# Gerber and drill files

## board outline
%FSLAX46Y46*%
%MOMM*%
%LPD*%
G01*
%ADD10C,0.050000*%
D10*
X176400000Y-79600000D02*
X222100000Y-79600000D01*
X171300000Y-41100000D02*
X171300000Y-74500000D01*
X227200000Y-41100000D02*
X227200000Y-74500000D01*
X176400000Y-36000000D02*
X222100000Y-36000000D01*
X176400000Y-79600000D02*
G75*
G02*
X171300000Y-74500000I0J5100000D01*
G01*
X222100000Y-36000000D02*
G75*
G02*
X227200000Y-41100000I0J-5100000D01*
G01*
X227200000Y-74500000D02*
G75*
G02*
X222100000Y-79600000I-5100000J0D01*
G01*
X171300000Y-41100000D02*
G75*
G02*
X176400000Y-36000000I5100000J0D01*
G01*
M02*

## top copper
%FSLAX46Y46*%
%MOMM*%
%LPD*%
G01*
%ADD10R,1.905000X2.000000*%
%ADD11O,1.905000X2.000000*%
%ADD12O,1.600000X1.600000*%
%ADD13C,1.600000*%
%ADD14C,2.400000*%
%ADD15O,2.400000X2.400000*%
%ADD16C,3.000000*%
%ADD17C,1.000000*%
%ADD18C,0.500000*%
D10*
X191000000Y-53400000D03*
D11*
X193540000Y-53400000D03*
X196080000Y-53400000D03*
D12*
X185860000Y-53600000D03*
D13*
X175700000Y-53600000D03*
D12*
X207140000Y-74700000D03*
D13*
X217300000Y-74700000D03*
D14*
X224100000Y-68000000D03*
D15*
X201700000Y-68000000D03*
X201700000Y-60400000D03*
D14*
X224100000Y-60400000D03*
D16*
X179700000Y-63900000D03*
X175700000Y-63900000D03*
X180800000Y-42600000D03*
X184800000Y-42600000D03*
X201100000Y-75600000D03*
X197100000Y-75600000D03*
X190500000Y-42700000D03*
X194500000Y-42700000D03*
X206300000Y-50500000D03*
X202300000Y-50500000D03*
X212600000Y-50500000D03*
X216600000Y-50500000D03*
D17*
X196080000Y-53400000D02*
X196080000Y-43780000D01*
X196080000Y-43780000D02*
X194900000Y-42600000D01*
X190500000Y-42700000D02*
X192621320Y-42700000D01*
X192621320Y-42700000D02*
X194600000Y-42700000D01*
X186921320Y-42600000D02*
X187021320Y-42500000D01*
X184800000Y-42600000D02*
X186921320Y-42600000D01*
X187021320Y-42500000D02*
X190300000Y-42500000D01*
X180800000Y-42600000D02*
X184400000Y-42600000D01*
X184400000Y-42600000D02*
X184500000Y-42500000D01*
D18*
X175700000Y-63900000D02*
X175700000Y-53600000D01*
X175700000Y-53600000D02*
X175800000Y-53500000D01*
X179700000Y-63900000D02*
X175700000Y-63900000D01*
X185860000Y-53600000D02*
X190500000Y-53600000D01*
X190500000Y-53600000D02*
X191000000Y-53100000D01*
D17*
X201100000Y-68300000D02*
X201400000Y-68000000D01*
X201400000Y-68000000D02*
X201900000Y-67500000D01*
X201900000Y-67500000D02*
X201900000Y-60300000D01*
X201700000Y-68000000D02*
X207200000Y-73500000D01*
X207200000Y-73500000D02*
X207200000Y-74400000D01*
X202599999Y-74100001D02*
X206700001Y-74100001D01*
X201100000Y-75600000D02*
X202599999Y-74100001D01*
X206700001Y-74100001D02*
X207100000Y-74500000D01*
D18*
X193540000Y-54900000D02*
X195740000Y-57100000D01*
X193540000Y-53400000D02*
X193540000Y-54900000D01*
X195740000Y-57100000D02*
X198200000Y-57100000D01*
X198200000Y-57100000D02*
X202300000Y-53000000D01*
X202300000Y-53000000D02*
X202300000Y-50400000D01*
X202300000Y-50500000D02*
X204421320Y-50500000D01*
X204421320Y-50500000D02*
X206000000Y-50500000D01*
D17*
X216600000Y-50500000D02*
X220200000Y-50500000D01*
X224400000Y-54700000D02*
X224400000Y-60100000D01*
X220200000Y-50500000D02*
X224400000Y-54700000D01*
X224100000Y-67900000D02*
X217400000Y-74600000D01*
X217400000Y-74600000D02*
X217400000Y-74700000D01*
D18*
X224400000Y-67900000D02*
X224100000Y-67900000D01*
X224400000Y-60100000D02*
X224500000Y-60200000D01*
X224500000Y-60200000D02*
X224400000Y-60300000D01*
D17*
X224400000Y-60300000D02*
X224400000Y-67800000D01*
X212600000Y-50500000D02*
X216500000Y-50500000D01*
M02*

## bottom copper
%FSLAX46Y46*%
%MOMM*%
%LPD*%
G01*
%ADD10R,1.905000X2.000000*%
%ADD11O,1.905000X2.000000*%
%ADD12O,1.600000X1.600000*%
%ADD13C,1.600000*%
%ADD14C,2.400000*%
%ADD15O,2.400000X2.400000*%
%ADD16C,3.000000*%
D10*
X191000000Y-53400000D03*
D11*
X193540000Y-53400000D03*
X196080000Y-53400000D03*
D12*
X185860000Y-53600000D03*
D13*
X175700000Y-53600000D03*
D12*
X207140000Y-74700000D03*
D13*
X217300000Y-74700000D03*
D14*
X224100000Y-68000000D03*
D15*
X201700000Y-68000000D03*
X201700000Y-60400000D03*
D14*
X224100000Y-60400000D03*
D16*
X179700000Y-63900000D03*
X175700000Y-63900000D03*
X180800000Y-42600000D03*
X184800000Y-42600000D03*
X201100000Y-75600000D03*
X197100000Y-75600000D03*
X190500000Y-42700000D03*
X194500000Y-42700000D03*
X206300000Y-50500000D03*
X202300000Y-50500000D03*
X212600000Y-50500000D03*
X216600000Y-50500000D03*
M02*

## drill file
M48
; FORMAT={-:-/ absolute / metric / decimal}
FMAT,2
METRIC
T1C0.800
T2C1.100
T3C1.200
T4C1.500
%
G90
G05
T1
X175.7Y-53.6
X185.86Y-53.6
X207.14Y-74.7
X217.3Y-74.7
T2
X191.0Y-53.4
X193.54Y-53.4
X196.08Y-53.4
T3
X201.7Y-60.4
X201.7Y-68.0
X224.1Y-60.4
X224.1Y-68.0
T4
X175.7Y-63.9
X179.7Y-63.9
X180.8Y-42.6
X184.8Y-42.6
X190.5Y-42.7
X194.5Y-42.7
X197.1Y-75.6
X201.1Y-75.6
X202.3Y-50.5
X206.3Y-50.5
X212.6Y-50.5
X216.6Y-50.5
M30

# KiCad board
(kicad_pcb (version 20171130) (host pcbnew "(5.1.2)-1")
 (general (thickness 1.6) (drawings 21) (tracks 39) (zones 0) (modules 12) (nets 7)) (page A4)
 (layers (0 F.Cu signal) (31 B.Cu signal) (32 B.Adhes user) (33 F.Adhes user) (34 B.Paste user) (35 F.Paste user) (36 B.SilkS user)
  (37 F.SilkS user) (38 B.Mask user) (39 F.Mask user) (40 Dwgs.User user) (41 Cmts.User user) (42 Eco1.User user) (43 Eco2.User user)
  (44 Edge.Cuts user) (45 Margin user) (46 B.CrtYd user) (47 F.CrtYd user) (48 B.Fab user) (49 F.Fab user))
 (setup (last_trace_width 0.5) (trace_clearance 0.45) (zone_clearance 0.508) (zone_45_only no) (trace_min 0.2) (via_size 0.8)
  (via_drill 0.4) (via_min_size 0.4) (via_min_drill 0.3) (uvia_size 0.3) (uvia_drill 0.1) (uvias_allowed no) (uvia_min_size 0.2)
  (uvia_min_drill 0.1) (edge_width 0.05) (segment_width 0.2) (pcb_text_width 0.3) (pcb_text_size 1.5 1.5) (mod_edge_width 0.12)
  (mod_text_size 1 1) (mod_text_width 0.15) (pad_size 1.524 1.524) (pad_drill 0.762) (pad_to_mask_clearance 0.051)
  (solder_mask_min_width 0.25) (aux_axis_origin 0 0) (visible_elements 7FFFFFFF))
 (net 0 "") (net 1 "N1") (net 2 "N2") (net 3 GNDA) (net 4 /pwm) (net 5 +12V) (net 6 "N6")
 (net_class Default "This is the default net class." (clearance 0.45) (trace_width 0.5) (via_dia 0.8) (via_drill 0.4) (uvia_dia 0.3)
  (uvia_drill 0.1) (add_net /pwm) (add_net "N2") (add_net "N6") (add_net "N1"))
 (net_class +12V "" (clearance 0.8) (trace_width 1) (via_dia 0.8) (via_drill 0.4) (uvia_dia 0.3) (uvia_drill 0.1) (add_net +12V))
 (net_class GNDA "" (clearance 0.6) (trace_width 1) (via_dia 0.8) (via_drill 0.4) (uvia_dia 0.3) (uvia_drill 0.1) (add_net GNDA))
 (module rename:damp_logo (layer F.Cu) (at 217.8 40.1)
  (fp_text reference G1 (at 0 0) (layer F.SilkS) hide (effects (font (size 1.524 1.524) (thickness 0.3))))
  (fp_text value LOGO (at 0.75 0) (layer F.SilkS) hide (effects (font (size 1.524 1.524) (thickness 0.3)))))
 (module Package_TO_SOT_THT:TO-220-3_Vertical (layer F.Cu) (at 191 53.4)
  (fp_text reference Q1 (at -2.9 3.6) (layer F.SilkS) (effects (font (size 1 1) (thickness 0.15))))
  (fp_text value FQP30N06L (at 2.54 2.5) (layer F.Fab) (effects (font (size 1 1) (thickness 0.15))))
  (pad 1 thru_hole rect (at 0 0) (size 1.905 2) (drill 1.1) (layers *.Cu *.Mask) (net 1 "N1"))
  (pad 2 thru_hole oval (at 2.54 0) (size 1.905 2) (drill 1.1) (layers *.Cu *.Mask) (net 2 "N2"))
  (pad 3 thru_hole oval (at 5.08 0) (size 1.905 2) (drill 1.1) (layers *.Cu *.Mask) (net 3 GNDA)))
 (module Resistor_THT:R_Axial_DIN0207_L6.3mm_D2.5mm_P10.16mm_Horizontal (layer F.Cu) (at 175.7 53.6)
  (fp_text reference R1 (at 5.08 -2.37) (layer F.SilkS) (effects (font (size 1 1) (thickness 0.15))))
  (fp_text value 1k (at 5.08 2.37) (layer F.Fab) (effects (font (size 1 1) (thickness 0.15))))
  (pad 2 thru_hole oval (at 10.16 0) (size 1.6 1.6) (drill 0.8) (layers *.Cu *.Mask) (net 1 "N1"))
  (pad 1 thru_hole circle (at 0 0) (size 1.6 1.6) (drill 0.8) (layers *.Cu *.Mask) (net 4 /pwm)))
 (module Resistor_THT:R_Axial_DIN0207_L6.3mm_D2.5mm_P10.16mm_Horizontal (layer F.Cu) (at 217.3 74.7 180)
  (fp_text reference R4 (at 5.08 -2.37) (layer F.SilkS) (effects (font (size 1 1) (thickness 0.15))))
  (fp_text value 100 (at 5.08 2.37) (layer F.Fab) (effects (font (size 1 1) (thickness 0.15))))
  (pad 2 thru_hole oval (at 10.16 0 180) (size 1.6 1.6) (drill 0.8) (layers *.Cu *.Mask) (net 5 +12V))
  (pad 1 thru_hole circle (at 0 0 180) (size 1.6 1.6) (drill 0.8) (layers *.Cu *.Mask) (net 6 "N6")))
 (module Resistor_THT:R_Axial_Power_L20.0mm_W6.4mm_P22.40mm (layer F.Cu) (at 224.1 68 180)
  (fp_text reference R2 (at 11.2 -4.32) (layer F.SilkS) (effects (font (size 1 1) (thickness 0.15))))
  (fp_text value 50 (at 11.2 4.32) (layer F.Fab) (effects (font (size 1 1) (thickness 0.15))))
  (pad 1 thru_hole circle (at 0 0 180) (size 2.4 2.4) (drill 1.2) (layers *.Cu *.Mask) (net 6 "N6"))
  (pad 2 thru_hole oval (at 22.4 0 180) (size 2.4 2.4) (drill 1.2) (layers *.Cu *.Mask) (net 5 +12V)))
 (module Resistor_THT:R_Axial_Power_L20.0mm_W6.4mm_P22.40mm (layer F.Cu) (at 224.1 60.4 180)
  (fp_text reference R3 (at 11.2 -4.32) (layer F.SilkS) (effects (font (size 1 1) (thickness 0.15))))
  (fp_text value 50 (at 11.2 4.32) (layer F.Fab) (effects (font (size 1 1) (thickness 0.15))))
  (pad 2 thru_hole oval (at 22.4 0 180) (size 2.4 2.4) (drill 1.2) (layers *.Cu *.Mask) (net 5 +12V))
  (pad 1 thru_hole circle (at 0 0 180) (size 2.4 2.4) (drill 1.2) (layers *.Cu *.Mask) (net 6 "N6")))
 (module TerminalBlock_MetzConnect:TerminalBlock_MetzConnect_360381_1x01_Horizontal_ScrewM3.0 (layer F.Cu) (at 175.7 63.9)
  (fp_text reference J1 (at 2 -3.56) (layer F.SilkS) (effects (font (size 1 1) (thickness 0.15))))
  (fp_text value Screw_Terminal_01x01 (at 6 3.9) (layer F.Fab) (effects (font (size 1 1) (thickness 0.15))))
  (pad 1 thru_hole circle (at 4 0) (size 3 3) (drill 1.5) (layers *.Cu *.Mask) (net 4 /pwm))
  (pad 1 thru_hole circle (at 0 0) (size 3 3) (drill 1.5) (layers *.Cu *.Mask) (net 4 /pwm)))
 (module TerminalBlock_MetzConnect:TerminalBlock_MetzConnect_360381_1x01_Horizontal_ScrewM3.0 (layer F.Cu) (at 180.8 42.6)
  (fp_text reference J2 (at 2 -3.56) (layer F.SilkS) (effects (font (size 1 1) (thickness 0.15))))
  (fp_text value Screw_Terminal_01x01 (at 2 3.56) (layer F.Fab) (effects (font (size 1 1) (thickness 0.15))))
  (pad 1 thru_hole circle (at 0 0) (size 3 3) (drill 1.5) (layers *.Cu *.Mask) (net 3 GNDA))
  (pad 1 thru_hole circle (at 4 0) (size 3 3) (drill 1.5) (layers *.Cu *.Mask) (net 3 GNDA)))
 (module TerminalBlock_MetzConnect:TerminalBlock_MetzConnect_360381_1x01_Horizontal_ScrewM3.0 (layer F.Cu) (at 197.1 75.6)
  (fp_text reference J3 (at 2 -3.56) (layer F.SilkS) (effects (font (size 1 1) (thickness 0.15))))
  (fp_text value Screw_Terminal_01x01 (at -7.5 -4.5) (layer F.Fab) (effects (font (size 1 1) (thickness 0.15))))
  (pad 1 thru_hole circle (at 4 0) (size 3 3) (drill 1.5) (layers *.Cu *.Mask) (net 5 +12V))
  (pad 1 thru_hole circle (at 0 0) (size 3 3) (drill 1.5) (layers *.Cu *.Mask) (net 5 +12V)))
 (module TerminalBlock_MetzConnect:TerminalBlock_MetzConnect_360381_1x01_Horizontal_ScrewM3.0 (layer F.Cu) (at 190.5 42.7)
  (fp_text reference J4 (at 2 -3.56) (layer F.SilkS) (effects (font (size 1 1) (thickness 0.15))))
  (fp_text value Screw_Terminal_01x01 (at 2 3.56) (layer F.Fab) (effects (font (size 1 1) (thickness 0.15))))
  (pad 1 thru_hole circle (at 0 0) (size 3 3) (drill 1.5) (layers *.Cu *.Mask) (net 3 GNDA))
  (pad 1 thru_hole circle (at 4 0) (size 3 3) (drill 1.5) (layers *.Cu *.Mask) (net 3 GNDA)))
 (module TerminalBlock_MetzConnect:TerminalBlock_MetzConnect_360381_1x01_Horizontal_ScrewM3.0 (layer F.Cu) (at 202.3 50.5)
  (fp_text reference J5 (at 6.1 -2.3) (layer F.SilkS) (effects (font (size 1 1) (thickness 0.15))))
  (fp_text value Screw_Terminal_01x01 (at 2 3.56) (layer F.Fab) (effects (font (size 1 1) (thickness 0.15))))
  (pad 1 thru_hole circle (at 4 0) (size 3 3) (drill 1.5) (layers *.Cu *.Mask) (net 2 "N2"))
  (pad 1 thru_hole circle (at 0 0) (size 3 3) (drill 1.5) (layers *.Cu *.Mask) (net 2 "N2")))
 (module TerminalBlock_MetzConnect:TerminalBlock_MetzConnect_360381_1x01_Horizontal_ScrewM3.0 (layer F.Cu) (at 212.6 50.5)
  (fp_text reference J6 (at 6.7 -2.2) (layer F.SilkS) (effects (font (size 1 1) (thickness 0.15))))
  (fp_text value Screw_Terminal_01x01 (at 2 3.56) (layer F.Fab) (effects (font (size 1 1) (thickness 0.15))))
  (pad 1 thru_hole circle (at 0 0) (size 3 3) (drill 1.5) (layers *.Cu *.Mask) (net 6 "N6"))
  (pad 1 thru_hole circle (at 4 0) (size 3 3) (drill 1.5) (layers *.Cu *.Mask) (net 6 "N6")))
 (gr_line (start 176.4 79.6) (end 222.1 79.6) (layer Edge.Cuts) (width 0.05))
 (gr_line (start 171.3 41.1) (end 171.3 74.5) (layer Edge.Cuts) (width 0.05))
 (gr_line (start 227.2 41.1) (end 227.2 74.5) (layer Edge.Cuts) (width 0.05))
 (gr_line (start 176.4 36) (end 222.1 36) (layer Edge.Cuts) (width 0.05))
 (gr_arc (start 176.4 74.5) (end 171.3 74.5) (angle -90) (layer Edge.Cuts) (width 0.05))
 (gr_arc (start 222.1 41.1) (end 227.2 41.1) (angle -90) (layer Edge.Cuts) (width 0.05))
 (gr_arc (start 222.1 74.5) (end 222.1 79.6) (angle -90) (layer Edge.Cuts) (width 0.05))
 (gr_arc (start 176.4 41.1) (end 176.4 36) (angle -90) (layer Edge.Cuts) (width 0.05))
 (segment (start 196.08 53.4) (end 196.08 43.78) (width 1) (layer F.Cu) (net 3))
 (segment (start 196.08 43.78) (end 194.9 42.6) (width 1) (layer F.Cu) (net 3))
 (segment (start 190.5 42.7) (end 192.62132 42.7) (width 1) (layer F.Cu) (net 3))
 (segment (start 192.62132 42.7) (end 194.6 42.7) (width 1) (layer F.Cu) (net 3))
 (segment (start 186.92132 42.6) (end 187.02132 42.5) (width 1) (layer F.Cu) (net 3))
 (segment (start 184.8 42.6) (end 186.92132 42.6) (width 1) (layer F.Cu) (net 3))
 (segment (start 187.02132 42.5) (end 190.3 42.5) (width 1) (layer F.Cu) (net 3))
 (segment (start 180.8 42.6) (end 184.4 42.6) (width 1) (layer F.Cu) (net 3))
 (segment (start 184.4 42.6) (end 184.5 42.5) (width 1) (layer F.Cu) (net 3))
 (segment (start 175.7 63.9) (end 175.7 53.6) (width 0.5) (layer F.Cu) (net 4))
 (segment (start 175.7 53.6) (end 175.8 53.5) (width 0.5) (layer F.Cu) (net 4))
 (segment (start 179.7 63.9) (end 175.7 63.9) (width 0.5) (layer F.Cu) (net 4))
 (segment (start 185.86 53.6) (end 190.5 53.6) (width 0.5) (layer F.Cu) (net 1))
 (segment (start 190.5 53.6) (end 191 53.1) (width 0.5) (layer F.Cu) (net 1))
 (segment (start 201.1 68.3) (end 201.4 68) (width 1) (layer F.Cu) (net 5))
 (segment (start 201.4 68) (end 201.9 67.5) (width 1) (layer F.Cu) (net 5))
 (segment (start 201.9 67.5) (end 201.9 60.3) (width 1) (layer F.Cu) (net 5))
 (segment (start 201.7 68) (end 207.2 73.5) (width 1) (layer F.Cu) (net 5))
 (segment (start 207.2 73.5) (end 207.2 74.4) (width 1) (layer F.Cu) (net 5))
 (segment (start 202.599999 74.100001) (end 206.700001 74.100001) (width 1) (layer F.Cu) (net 5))
 (segment (start 201.1 75.6) (end 202.599999 74.100001) (width 1) (layer F.Cu) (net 5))
 (segment (start 206.700001 74.100001) (end 207.1 74.5) (width 1) (layer F.Cu) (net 5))
 (segment (start 193.54 54.9) (end 195.74 57.1) (width 0.5) (layer F.Cu) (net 2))
 (segment (start 193.54 53.4) (end 193.54 54.9) (width 0.5) (layer F.Cu) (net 2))
 (segment (start 195.74 57.1) (end 198.2 57.1) (width 0.5) (layer F.Cu) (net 2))
 (segment (start 198.2 57.1) (end 202.3 53) (width 0.5) (layer F.Cu) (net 2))
 (segment (start 202.3 53) (end 202.3 50.4) (width 0.5) (layer F.Cu) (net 2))
 (segment (start 202.3 50.5) (end 204.42132 50.5) (width 0.5) (layer F.Cu) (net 2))
 (segment (start 204.42132 50.5) (end 206 50.5) (width 0.5) (layer F.Cu) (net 2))
 (segment (start 216.6 50.5) (end 220.2 50.5) (width 1) (layer F.Cu) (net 6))
 (segment (start 224.4 54.7) (end 224.4 60.1) (width 1) (layer F.Cu) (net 6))
 (segment (start 220.2 50.5) (end 224.4 54.7) (width 1) (layer F.Cu) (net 6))
 (segment (start 224.1 67.9) (end 217.4 74.6) (width 1) (layer F.Cu) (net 6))
 (segment (start 217.4 74.6) (end 217.4 74.7) (width 1) (layer F.Cu) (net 6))
 (segment (start 224.4 67.9) (end 224.1 67.9) (width 0.5) (layer F.Cu) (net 6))
 (segment (start 224.4 60.1) (end 224.5 60.2) (width 0.5) (layer F.Cu) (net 6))
 (segment (start 224.5 60.2) (end 224.4 60.3) (width 0.5) (layer F.Cu) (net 6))
 (segment (start 224.4 60.3) (end 224.4 67.8) (width 1) (layer F.Cu) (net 6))
 (segment (start 212.6 50.5) (end 216.5 50.5) (width 1) (layer F.Cu) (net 6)))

